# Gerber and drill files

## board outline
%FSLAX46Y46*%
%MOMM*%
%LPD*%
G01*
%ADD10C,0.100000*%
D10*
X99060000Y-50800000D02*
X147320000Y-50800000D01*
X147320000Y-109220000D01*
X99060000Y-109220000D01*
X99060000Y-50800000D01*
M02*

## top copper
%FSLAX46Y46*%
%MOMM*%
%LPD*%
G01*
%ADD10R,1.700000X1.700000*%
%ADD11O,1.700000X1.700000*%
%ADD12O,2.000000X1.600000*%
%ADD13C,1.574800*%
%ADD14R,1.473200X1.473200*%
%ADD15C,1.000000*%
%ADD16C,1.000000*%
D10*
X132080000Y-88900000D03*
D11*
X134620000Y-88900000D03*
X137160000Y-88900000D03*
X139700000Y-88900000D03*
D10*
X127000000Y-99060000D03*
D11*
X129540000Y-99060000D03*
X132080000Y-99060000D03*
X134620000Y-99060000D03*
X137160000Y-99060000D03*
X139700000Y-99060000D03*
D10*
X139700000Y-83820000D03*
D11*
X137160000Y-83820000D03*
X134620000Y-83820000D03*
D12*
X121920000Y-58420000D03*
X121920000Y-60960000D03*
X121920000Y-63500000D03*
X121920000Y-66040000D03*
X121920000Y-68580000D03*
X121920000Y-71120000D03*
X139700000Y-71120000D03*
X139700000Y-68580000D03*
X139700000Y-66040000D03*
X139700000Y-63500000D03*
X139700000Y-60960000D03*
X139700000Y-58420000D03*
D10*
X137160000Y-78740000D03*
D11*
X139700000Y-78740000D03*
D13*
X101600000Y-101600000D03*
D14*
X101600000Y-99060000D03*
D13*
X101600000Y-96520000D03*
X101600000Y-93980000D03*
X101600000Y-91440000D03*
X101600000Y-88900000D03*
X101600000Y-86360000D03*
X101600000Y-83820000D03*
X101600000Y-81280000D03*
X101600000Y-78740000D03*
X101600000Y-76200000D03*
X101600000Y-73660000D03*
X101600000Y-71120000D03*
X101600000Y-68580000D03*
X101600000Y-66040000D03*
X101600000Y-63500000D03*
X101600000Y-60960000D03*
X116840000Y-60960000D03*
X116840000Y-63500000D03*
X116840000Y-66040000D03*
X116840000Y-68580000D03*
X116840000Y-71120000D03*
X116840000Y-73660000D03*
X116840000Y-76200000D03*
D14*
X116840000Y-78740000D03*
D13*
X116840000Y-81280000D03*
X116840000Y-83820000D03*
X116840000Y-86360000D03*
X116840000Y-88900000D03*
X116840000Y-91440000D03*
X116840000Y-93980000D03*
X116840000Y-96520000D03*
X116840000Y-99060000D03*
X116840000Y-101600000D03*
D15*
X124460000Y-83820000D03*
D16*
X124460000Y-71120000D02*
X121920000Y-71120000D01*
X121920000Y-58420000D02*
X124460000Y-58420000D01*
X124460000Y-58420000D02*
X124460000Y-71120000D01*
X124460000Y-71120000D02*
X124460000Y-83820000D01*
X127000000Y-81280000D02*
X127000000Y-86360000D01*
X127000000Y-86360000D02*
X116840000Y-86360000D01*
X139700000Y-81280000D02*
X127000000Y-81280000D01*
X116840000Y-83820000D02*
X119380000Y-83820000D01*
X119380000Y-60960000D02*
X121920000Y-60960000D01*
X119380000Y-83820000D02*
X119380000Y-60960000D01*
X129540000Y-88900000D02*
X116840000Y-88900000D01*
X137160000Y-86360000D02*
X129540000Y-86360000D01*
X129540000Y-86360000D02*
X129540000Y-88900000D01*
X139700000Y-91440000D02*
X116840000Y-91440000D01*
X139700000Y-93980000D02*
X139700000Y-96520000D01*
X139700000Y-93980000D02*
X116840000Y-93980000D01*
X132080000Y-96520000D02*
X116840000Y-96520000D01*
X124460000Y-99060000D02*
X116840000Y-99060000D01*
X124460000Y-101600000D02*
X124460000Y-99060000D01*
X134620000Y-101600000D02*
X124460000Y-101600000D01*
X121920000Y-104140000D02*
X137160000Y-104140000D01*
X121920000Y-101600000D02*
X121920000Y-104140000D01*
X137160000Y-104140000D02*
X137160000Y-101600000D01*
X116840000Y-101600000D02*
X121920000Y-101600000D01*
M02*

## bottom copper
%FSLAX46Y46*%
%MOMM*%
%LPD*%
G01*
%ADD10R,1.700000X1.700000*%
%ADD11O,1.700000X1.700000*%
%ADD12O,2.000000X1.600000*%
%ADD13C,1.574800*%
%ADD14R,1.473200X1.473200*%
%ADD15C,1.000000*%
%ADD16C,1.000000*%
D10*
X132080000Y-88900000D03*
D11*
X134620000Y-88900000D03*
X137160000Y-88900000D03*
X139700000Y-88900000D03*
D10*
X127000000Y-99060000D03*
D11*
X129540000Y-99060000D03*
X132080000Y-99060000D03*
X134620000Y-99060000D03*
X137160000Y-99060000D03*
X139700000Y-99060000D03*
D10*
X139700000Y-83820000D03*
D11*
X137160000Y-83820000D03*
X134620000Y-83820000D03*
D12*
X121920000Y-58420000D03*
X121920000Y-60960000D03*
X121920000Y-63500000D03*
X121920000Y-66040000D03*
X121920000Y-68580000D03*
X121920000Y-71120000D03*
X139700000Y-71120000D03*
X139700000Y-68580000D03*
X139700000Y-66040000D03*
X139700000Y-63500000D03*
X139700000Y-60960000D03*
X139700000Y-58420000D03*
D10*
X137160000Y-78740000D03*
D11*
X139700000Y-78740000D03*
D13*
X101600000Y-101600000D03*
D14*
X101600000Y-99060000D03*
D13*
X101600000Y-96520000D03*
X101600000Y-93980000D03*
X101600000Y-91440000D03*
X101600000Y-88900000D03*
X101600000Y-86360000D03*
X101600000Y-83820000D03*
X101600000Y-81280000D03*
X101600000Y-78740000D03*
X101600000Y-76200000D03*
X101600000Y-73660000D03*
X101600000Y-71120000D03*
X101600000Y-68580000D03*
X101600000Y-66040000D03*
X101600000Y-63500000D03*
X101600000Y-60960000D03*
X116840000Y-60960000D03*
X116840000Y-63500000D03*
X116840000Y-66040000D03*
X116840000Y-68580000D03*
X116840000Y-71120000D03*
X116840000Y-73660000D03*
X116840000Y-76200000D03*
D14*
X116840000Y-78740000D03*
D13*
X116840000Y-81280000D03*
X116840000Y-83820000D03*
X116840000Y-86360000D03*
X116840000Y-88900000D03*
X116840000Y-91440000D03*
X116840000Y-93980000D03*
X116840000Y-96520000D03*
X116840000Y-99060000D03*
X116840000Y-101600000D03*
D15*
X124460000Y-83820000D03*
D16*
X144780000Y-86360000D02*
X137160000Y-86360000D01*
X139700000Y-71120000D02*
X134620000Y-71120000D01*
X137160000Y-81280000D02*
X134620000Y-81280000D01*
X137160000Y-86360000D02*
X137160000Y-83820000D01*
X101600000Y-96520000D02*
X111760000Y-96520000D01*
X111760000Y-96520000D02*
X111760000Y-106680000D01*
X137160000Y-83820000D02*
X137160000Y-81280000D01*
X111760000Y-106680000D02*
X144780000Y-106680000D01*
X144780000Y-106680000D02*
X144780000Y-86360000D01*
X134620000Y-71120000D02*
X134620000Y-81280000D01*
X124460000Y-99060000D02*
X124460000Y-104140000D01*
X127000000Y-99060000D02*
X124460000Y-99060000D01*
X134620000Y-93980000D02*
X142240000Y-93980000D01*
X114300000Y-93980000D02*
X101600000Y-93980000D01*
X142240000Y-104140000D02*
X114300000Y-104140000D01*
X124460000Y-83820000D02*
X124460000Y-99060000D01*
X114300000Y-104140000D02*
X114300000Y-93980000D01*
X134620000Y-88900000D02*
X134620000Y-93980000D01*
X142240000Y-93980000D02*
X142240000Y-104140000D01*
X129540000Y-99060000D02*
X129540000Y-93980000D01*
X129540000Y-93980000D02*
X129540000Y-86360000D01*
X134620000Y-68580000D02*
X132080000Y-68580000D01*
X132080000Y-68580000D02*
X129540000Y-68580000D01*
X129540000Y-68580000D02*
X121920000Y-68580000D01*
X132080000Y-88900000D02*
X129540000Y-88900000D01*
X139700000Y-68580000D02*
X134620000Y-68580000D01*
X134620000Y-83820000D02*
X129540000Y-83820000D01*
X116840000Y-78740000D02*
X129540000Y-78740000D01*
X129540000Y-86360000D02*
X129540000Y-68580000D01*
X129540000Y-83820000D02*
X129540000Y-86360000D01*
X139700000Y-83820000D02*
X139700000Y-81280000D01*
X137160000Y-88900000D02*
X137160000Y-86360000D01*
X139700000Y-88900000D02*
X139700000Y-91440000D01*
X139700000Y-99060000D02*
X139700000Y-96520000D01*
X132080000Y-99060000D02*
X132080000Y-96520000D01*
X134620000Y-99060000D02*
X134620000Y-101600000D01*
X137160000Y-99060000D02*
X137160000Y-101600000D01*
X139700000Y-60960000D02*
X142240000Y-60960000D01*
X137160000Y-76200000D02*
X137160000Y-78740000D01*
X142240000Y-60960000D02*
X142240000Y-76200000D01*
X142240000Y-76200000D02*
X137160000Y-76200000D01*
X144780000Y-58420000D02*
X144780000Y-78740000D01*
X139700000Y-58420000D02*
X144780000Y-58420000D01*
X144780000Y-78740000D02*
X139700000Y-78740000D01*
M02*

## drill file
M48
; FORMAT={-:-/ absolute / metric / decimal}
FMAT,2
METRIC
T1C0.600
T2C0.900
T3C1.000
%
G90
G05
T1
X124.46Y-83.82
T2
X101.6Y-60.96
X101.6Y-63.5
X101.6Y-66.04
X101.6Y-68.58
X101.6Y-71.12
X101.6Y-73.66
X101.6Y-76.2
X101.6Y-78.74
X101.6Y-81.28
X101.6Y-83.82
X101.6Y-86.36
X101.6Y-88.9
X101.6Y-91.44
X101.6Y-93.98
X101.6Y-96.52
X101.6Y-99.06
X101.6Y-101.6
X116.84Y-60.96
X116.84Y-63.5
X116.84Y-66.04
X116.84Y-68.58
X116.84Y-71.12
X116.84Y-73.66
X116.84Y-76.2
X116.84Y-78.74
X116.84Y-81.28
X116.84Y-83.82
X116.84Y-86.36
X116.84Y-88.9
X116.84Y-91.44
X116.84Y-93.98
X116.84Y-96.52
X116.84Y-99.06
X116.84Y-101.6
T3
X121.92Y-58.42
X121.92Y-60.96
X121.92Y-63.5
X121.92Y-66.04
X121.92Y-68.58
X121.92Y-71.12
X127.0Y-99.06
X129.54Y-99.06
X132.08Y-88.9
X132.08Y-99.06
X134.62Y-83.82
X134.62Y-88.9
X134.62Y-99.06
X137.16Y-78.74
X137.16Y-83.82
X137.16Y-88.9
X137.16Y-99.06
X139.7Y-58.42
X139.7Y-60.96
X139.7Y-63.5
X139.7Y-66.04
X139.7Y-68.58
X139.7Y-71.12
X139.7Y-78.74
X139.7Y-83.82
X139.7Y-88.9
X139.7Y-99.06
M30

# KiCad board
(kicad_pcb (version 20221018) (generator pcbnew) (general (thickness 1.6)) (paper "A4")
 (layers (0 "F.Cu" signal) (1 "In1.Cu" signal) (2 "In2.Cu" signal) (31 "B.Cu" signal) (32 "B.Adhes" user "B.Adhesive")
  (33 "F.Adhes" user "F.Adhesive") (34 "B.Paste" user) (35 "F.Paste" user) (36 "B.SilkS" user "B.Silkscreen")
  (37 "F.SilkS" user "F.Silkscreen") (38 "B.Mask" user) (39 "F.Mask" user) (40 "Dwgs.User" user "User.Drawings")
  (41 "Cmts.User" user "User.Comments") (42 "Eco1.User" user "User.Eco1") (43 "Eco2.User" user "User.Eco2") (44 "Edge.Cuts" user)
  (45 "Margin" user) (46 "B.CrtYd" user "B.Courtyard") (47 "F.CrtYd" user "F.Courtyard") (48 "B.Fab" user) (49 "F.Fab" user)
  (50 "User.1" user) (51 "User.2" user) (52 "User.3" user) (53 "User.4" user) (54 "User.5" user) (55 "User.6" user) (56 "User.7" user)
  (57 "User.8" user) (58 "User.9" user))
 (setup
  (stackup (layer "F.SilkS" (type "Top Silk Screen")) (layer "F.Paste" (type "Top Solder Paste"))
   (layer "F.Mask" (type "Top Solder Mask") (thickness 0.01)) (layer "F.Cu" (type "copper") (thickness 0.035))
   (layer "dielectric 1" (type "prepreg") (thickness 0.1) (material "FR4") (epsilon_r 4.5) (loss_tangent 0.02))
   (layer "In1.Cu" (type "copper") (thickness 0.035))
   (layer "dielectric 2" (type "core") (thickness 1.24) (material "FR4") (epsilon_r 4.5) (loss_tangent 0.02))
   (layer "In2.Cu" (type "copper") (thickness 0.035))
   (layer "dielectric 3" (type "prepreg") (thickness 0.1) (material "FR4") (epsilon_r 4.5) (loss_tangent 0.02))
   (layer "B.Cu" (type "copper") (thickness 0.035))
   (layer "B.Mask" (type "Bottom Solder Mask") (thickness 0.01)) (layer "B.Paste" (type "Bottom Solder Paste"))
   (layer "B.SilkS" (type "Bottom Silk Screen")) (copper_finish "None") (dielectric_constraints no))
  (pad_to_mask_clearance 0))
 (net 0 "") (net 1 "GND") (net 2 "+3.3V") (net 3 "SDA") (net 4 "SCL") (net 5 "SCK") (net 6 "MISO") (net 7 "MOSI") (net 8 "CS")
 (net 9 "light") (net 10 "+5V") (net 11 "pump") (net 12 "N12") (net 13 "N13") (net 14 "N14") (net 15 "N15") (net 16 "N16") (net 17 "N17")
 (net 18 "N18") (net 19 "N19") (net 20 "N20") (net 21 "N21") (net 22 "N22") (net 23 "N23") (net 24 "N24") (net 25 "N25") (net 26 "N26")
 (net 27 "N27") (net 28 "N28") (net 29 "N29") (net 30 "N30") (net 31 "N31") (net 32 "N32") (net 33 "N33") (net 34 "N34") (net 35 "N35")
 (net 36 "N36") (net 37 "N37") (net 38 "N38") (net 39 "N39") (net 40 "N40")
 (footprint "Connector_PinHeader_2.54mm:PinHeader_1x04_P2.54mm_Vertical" (layer "F.Cu") (at 132.08 88.9 90)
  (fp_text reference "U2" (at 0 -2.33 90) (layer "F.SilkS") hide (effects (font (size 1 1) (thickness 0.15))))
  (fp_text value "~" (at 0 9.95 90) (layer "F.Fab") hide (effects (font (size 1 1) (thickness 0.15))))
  (pad "1" thru_hole rect (at 0 0 90) (size 1.7 1.7) (drill 1) (layers "*.Cu" "*.Mask") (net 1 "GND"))
  (pad "2" thru_hole oval (at 0 2.54 90) (size 1.7 1.7) (drill 1) (layers "*.Cu" "*.Mask") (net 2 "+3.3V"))
  (pad "3" thru_hole oval (at 0 5.08 90) (size 1.7 1.7) (drill 1) (layers "*.Cu" "*.Mask") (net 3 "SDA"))
  (pad "4" thru_hole oval (at 0 7.62 90) (size 1.7 1.7) (drill 1) (layers "*.Cu" "*.Mask") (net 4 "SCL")))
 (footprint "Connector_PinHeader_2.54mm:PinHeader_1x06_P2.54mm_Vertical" (layer "F.Cu") (at 127 99.06 90)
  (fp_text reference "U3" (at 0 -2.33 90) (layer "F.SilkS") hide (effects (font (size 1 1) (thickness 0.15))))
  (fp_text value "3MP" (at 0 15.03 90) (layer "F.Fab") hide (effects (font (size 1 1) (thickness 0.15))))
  (pad "1" thru_hole rect (at 0 0 90) (size 1.7 1.7) (drill 1) (layers "*.Cu" "*.Mask") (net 2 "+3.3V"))
  (pad "2" thru_hole oval (at 0 2.54 90) (size 1.7 1.7) (drill 1) (layers "*.Cu" "*.Mask") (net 1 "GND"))
  (pad "3" thru_hole oval (at 0 5.08 90) (size 1.7 1.7) (drill 1) (layers "*.Cu" "*.Mask") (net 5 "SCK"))
  (pad "4" thru_hole oval (at 0 7.62 90) (size 1.7 1.7) (drill 1) (layers "*.Cu" "*.Mask") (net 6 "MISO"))
  (pad "5" thru_hole oval (at 0 10.16 90) (size 1.7 1.7) (drill 1) (layers "*.Cu" "*.Mask") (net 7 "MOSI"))
  (pad "6" thru_hole oval (at 0 12.7 90) (size 1.7 1.7) (drill 1) (layers "*.Cu" "*.Mask") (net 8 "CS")))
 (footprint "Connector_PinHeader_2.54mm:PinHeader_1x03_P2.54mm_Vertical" (layer "F.Cu") (at 139.7 83.82 -90)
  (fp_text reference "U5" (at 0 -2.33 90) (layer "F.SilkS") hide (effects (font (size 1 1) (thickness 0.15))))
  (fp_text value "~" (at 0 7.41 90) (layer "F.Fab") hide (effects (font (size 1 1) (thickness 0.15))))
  (pad "1" thru_hole rect (at 0 0 270) (size 1.7 1.7) (drill 1) (layers "*.Cu" "*.Mask") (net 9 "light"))
  (pad "2" thru_hole oval (at 0 2.54 270) (size 1.7 1.7) (drill 1) (layers "*.Cu" "*.Mask") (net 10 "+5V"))
  (pad "3" thru_hole oval (at 0 5.08 270) (size 1.7 1.7) (drill 1) (layers "*.Cu" "*.Mask") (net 1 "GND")))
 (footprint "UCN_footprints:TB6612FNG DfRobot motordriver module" (layer "F.Cu") (at 121.92 58.42)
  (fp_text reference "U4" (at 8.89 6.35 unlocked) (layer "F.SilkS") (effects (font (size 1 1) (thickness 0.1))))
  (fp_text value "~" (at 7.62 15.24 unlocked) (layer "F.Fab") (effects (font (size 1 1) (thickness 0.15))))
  (pad "1" thru_hole oval (at 0 0 90) (size 1.6 2) (drill 1) (layers "*.Cu" "*.Mask") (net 2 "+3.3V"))
  (pad "2" thru_hole oval (at 0 2.54 90) (size 1.6 2) (drill 1) (layers "*.Cu" "*.Mask") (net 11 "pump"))
  (pad "3" thru_hole oval (at 0 5.08 90) (size 1.6 2) (drill 1) (layers "*.Cu" "*.Mask") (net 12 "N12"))
  (pad "4" thru_hole oval (at 0 7.62 90) (size 1.6 2) (drill 1) (layers "*.Cu" "*.Mask") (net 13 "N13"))
  (pad "5" thru_hole oval (at 0 10.16 90) (size 1.6 2) (drill 1) (layers "*.Cu" "*.Mask") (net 1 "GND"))
  (pad "6" thru_hole oval (at 0 12.7 90) (size 1.6 2) (drill 1) (layers "*.Cu" "*.Mask") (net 2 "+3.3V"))
  (pad "7" thru_hole oval (at 17.78 12.7 90) (size 1.6 2) (drill 1) (layers "*.Cu" "*.Mask") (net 10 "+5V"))
  (pad "8" thru_hole oval (at 17.78 10.16 90) (size 1.6 2) (drill 1) (layers "*.Cu" "*.Mask") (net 1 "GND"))
  (pad "9" thru_hole oval (at 17.78 7.62 90) (size 1.6 2) (drill 1) (layers "*.Cu" "*.Mask") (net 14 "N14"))
  (pad "10" thru_hole oval (at 17.78 5.08 90) (size 1.6 2) (drill 1) (layers "*.Cu" "*.Mask") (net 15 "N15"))
  (pad "11" thru_hole oval (at 17.78 2.54 90) (size 1.6 2) (drill 1) (layers "*.Cu" "*.Mask") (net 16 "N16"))
  (pad "12" thru_hole oval (at 17.78 0 90) (size 1.6 2) (drill 1) (layers "*.Cu" "*.Mask") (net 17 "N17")))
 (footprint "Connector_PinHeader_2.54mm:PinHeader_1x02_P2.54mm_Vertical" (layer "F.Cu") (at 137.16 78.74 90)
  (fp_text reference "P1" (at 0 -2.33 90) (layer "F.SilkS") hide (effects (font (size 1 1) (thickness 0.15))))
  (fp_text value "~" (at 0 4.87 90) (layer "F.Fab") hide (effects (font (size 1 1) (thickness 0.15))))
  (pad "1" thru_hole rect (at 0 0 90) (size 1.7 1.7) (drill 1) (layers "*.Cu" "*.Mask") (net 16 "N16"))
  (pad "2" thru_hole oval (at 0 2.54 90) (size 1.7 1.7) (drill 1) (layers "*.Cu" "*.Mask") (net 17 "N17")))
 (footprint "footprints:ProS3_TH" (layer "F.Cu") (at 109.2 81.28 180)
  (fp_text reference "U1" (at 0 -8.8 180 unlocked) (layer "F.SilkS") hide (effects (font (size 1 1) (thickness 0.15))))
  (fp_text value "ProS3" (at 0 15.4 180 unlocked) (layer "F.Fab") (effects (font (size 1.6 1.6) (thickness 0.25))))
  (pad "1" thru_hole circle (at 7.6 -20.32 180) (size 1.5748 1.5748) (drill 0.9) (layers "*.Cu" "*.Mask") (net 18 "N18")
   (solder_mask_margin 0.0254))
  (pad "2" thru_hole rect (at 7.6 -17.78 180) (size 1.4732 1.4732) (drill 0.9) (layers "*.Cu" "*.Mask") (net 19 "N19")
   (solder_mask_margin 0.0254))
  (pad "3" thru_hole circle (at 7.6 -15.24 180) (size 1.5748 1.5748) (drill 0.9) (layers "*.Cu" "*.Mask") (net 10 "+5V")
   (solder_mask_margin 0.0254))
  (pad "4" thru_hole circle (at 7.6 -12.7 180) (size 1.5748 1.5748) (drill 0.9) (layers "*.Cu" "*.Mask") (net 2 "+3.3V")
   (solder_mask_margin 0.0254))
  (pad "5" thru_hole circle (at 7.6 -10.16 180) (size 1.5748 1.5748) (drill 0.9) (layers "*.Cu" "*.Mask") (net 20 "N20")
   (solder_mask_margin 0.0254))
  (pad "6" thru_hole circle (at 7.6 -7.62 180) (size 1.5748 1.5748) (drill 0.9) (layers "*.Cu" "*.Mask") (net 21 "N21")
   (solder_mask_margin 0.0254))
  (pad "7" thru_hole circle (at 7.6 -5.08 180) (size 1.5748 1.5748) (drill 0.9) (layers "*.Cu" "*.Mask") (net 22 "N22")
   (solder_mask_margin 0.0254))
  (pad "8" thru_hole circle (at 7.6 -2.54 180) (size 1.5748 1.5748) (drill 0.9) (layers "*.Cu" "*.Mask") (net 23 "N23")
   (solder_mask_margin 0.0254))
  (pad "9" thru_hole circle (at 7.6 0 180) (size 1.5748 1.5748) (drill 0.9) (layers "*.Cu" "*.Mask") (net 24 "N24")
   (solder_mask_margin 0.0254))
  (pad "10" thru_hole circle (at 7.6 2.54 180) (size 1.5748 1.5748) (drill 0.9) (layers "*.Cu" "*.Mask") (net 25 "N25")
   (solder_mask_margin 0.0254))
  (pad "11" thru_hole circle (at 7.6 5.08 180) (size 1.5748 1.5748) (drill 0.9) (layers "*.Cu" "*.Mask") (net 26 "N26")
   (solder_mask_margin 0.0254))
  (pad "12" thru_hole circle (at 7.6 7.62 180) (size 1.5748 1.5748) (drill 0.9) (layers "*.Cu" "*.Mask") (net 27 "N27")
   (solder_mask_margin 0.0254))
  (pad "13" thru_hole circle (at 7.6 10.16 180) (size 1.5748 1.5748) (drill 0.9) (layers "*.Cu" "*.Mask") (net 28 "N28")
   (solder_mask_margin 0.0254))
  (pad "14" thru_hole circle (at 7.6 12.7 180) (size 1.5748 1.5748) (drill 0.9) (layers "*.Cu" "*.Mask") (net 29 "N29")
   (solder_mask_margin 0.0254))
  (pad "15" thru_hole circle (at 7.6 15.24 180) (size 1.5748 1.5748) (drill 0.9) (layers "*.Cu" "*.Mask") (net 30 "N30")
   (solder_mask_margin 0.0254))
  (pad "16" thru_hole circle (at 7.6 17.78 180) (size 1.5748 1.5748) (drill 0.9) (layers "*.Cu" "*.Mask") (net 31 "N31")
   (solder_mask_margin 0.0254))
  (pad "17" thru_hole circle (at 7.6 20.32 180) (size 1.5748 1.5748) (drill 0.9) (layers "*.Cu" "*.Mask") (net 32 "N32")
   (solder_mask_margin 0.0254))
  (pad "18" thru_hole circle (at -7.64 20.32 180) (size 1.5748 1.5748) (drill 0.9) (layers "*.Cu" "*.Mask") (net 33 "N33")
   (solder_mask_margin 0.0254))
  (pad "19" thru_hole circle (at -7.64 17.78 180) (size 1.5748 1.5748) (drill 0.9) (layers "*.Cu" "*.Mask") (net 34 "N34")
   (solder_mask_margin 0.0254))
  (pad "20" thru_hole circle (at -7.64 15.24 180) (size 1.5748 1.5748) (drill 0.9) (layers "*.Cu" "*.Mask") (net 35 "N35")
   (solder_mask_margin 0.0254))
  (pad "21" thru_hole circle (at -7.64 12.7 180) (size 1.5748 1.5748) (drill 0.9) (layers "*.Cu" "*.Mask") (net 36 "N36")
   (solder_mask_margin 0.0254))
  (pad "22" thru_hole circle (at -7.64 10.16 180) (size 1.5748 1.5748) (drill 0.9) (layers "*.Cu" "*.Mask") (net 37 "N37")
   (solder_mask_margin 0.0254))
  (pad "23" thru_hole circle (at -7.64 7.62 180) (size 1.5748 1.5748) (drill 0.9) (layers "*.Cu" "*.Mask") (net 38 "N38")
   (solder_mask_margin 0.0254))
  (pad "24" thru_hole circle (at -7.64 5.08 180) (size 1.5748 1.5748) (drill 0.9) (layers "*.Cu" "*.Mask") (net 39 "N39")
   (solder_mask_margin 0.0254))
  (pad "25" thru_hole rect (at -7.64 2.54 180) (size 1.4732 1.4732) (drill 0.9) (layers "*.Cu" "*.Mask") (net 1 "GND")
   (solder_mask_margin 0.0254))
  (pad "26" thru_hole circle (at -7.64 0 180) (size 1.5748 1.5748) (drill 0.9) (layers "*.Cu" "*.Mask") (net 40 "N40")
   (solder_mask_margin 0.0254))
  (pad "27" thru_hole circle (at -7.64 -2.54 180) (size 1.5748 1.5748) (drill 0.9) (layers "*.Cu" "*.Mask") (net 11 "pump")
   (solder_mask_margin 0.0254))
  (pad "28" thru_hole circle (at -7.64 -5.08 180) (size 1.5748 1.5748) (drill 0.9) (layers "*.Cu" "*.Mask") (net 9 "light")
   (solder_mask_margin 0.0254))
  (pad "29" thru_hole circle (at -7.64 -7.62 180) (size 1.5748 1.5748) (drill 0.9) (layers "*.Cu" "*.Mask") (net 3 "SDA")
   (solder_mask_margin 0.0254))
  (pad "30" thru_hole circle (at -7.64 -10.16 180) (size 1.5748 1.5748) (drill 0.9) (layers "*.Cu" "*.Mask") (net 4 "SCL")
   (solder_mask_margin 0.0254))
  (pad "31" thru_hole circle (at -7.64 -12.7 180) (size 1.5748 1.5748) (drill 0.9) (layers "*.Cu" "*.Mask") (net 8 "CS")
   (solder_mask_margin 0.0254))
  (pad "32" thru_hole circle (at -7.64 -15.24 180) (size 1.5748 1.5748) (drill 0.9) (layers "*.Cu" "*.Mask") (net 5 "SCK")
   (solder_mask_margin 0.0254))
  (pad "33" thru_hole circle (at -7.64 -17.78 180) (size 1.5748 1.5748) (drill 0.9) (layers "*.Cu" "*.Mask") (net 6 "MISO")
   (solder_mask_margin 0.0254))
  (pad "34" thru_hole circle (at -7.64 -20.32 180) (size 1.5748 1.5748) (drill 0.9) (layers "*.Cu" "*.Mask") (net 7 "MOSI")
   (solder_mask_margin 0.0254)))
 (gr_rect (start 99.06 50.8) (end 147.32 109.22) (stroke (width 0.1) (type default)) (fill none) (layer "Edge.Cuts"))
 (segment (start 144.78 86.36) (end 137.16 86.36) (width 1) (layer "B.Cu") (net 10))
 (segment (start 139.7 71.12) (end 134.62 71.12) (width 1) (layer "B.Cu") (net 10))
 (segment (start 137.16 81.28) (end 134.62 81.28) (width 1) (layer "B.Cu") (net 10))
 (segment (start 137.16 86.36) (end 137.16 83.82) (width 1) (layer "B.Cu") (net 10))
 (segment (start 101.6 96.52) (end 111.76 96.52) (width 1) (layer "B.Cu") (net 10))
 (segment (start 111.76 96.52) (end 111.76 106.68) (width 1) (layer "B.Cu") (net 10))
 (segment (start 137.16 83.82) (end 137.16 81.28) (width 1) (layer "B.Cu") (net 10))
 (segment (start 111.76 106.68) (end 144.78 106.68) (width 1) (layer "B.Cu") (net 10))
 (segment (start 144.78 106.68) (end 144.78 86.36) (width 1) (layer "B.Cu") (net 10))
 (segment (start 134.62 71.12) (end 134.62 81.28) (width 1) (layer "B.Cu") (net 10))
 (segment (start 124.46 71.12) (end 121.92 71.12) (width 1) (layer "F.Cu") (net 2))
 (segment (start 121.92 58.42) (end 124.46 58.42) (width 1) (layer "F.Cu") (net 2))
 (segment (start 124.46 58.42) (end 124.46 71.12) (width 1) (layer "F.Cu") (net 2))
 (segment (start 124.46 71.12) (end 124.46 83.82) (width 1) (layer "F.Cu") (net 2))
 (via (at 124.46 83.82) (size 1) (drill 0.6) (layers "F.Cu" "B.Cu") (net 2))
 (segment (start 124.46 99.06) (end 124.46 104.14) (width 1) (layer "B.Cu") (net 2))
 (segment (start 127 99.06) (end 124.46 99.06) (width 1) (layer "B.Cu") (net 2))
 (segment (start 134.62 93.98) (end 142.24 93.98) (width 1) (layer "B.Cu") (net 2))
 (segment (start 114.3 93.98) (end 101.6 93.98) (width 1) (layer "B.Cu") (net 2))
 (segment (start 142.24 104.14) (end 114.3 104.14) (width 1) (layer "B.Cu") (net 2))
 (segment (start 124.46 83.82) (end 124.46 99.06) (width 1) (layer "B.Cu") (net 2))
 (segment (start 114.3 104.14) (end 114.3 93.98) (width 1) (layer "B.Cu") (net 2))
 (segment (start 134.62 88.9) (end 134.62 93.98) (width 1) (layer "B.Cu") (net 2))
 (segment (start 142.24 93.98) (end 142.24 104.14) (width 1) (layer "B.Cu") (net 2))
 (segment (start 129.54 99.06) (end 129.54 93.98) (width 1) (layer "B.Cu") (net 1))
 (segment (start 129.54 93.98) (end 129.54 86.36) (width 1) (layer "B.Cu") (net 1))
 (segment (start 134.62 68.58) (end 132.08 68.58) (width 1) (layer "B.Cu") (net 1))
 (segment (start 132.08 68.58) (end 129.54 68.58) (width 1) (layer "B.Cu") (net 1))
 (segment (start 129.54 68.58) (end 121.92 68.58) (width 1) (layer "B.Cu") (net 1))
 (segment (start 132.08 88.9) (end 129.54 88.9) (width 1) (layer "B.Cu") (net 1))
 (segment (start 139.7 68.58) (end 134.62 68.58) (width 1) (layer "B.Cu") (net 1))
 (segment (start 134.62 83.82) (end 129.54 83.82) (width 1) (layer "B.Cu") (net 1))
 (segment (start 116.84 78.74) (end 129.54 78.74) (width 1) (layer "B.Cu") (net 1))
 (segment (start 129.54 86.36) (end 129.54 68.58) (width 1) (layer "B.Cu") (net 1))
 (segment (start 129.54 83.82) (end 129.54 86.36) (width 1) (layer "B.Cu") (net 1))
 (segment (start 127 81.28) (end 127 86.36) (width 1) (layer "F.Cu") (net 9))
 (segment (start 127 86.36) (end 116.84 86.36) (width 1) (layer "F.Cu") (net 9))
 (segment (start 139.7 81.28) (end 127 81.28) (width 1) (layer "F.Cu") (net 9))
 (segment (start 139.7 83.82) (end 139.7 81.28) (width 1) (layer "B.Cu") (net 9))
 (segment (start 116.84 83.82) (end 119.38 83.82) (width 1) (layer "F.Cu") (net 11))
 (segment (start 119.38 60.96) (end 121.92 60.96) (width 1) (layer "F.Cu") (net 11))
 (segment (start 119.38 83.82) (end 119.38 60.96) (width 1) (layer "F.Cu") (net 11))
 (segment (start 129.54 88.9) (end 116.84 88.9) (width 1) (layer "F.Cu") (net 3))
 (segment (start 137.16 86.36) (end 129.54 86.36) (width 1) (layer "F.Cu") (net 3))
 (segment (start 129.54 86.36) (end 129.54 88.9) (width 1) (layer "F.Cu") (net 3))
 (segment (start 137.16 88.9) (end 137.16 86.36) (width 1) (layer "B.Cu") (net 3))
 (segment (start 139.7 91.44) (end 116.84 91.44) (width 1) (layer "F.Cu") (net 4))
 (segment (start 139.7 88.9) (end 139.7 91.44) (width 1) (layer "B.Cu") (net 4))
 (segment (start 139.7 93.98) (end 139.7 96.52) (width 1) (layer "F.Cu") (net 8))
 (segment (start 139.7 93.98) (end 116.84 93.98) (width 1) (layer "F.Cu") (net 8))
 (segment (start 139.7 99.06) (end 139.7 96.52) (width 1) (layer "B.Cu") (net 8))
 (segment (start 132.08 96.52) (end 116.84 96.52) (width 1) (layer "F.Cu") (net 5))
 (segment (start 132.08 99.06) (end 132.08 96.52) (width 1) (layer "B.Cu") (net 5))
 (segment (start 124.46 99.06) (end 116.84 99.06) (width 1) (layer "F.Cu") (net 6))
 (segment (start 124.46 101.6) (end 124.46 99.06) (width 1) (layer "F.Cu") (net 6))
 (segment (start 134.62 101.6) (end 124.46 101.6) (width 1) (layer "F.Cu") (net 6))
 (segment (start 134.62 99.06) (end 134.62 101.6) (width 1) (layer "B.Cu") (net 6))
 (segment (start 121.92 104.14) (end 137.16 104.14) (width 1) (layer "F.Cu") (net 7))
 (segment (start 121.92 101.6) (end 121.92 104.14) (width 1) (layer "F.Cu") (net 7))
 (segment (start 137.16 104.14) (end 137.16 101.6) (width 1) (layer "F.Cu") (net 7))
 (segment (start 116.84 101.6) (end 121.92 101.6) (width 1) (layer "F.Cu") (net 7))
 (segment (start 137.16 99.06) (end 137.16 101.6) (width 1) (layer "B.Cu") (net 7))
 (segment (start 139.7 60.96) (end 142.24 60.96) (width 1) (layer "B.Cu") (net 16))
 (segment (start 137.16 76.2) (end 137.16 78.74) (width 1) (layer "B.Cu") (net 16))
 (segment (start 142.24 60.96) (end 142.24 76.2) (width 1) (layer "B.Cu") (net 16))
 (segment (start 142.24 76.2) (end 137.16 76.2) (width 1) (layer "B.Cu") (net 16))
 (segment (start 144.78 58.42) (end 144.78 78.74) (width 1) (layer "B.Cu") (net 17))
 (segment (start 139.7 58.42) (end 144.78 58.42) (width 1) (layer "B.Cu") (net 17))
 (segment (start 144.78 78.74) (end 139.7 78.74) (width 1) (layer "B.Cu") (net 17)))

